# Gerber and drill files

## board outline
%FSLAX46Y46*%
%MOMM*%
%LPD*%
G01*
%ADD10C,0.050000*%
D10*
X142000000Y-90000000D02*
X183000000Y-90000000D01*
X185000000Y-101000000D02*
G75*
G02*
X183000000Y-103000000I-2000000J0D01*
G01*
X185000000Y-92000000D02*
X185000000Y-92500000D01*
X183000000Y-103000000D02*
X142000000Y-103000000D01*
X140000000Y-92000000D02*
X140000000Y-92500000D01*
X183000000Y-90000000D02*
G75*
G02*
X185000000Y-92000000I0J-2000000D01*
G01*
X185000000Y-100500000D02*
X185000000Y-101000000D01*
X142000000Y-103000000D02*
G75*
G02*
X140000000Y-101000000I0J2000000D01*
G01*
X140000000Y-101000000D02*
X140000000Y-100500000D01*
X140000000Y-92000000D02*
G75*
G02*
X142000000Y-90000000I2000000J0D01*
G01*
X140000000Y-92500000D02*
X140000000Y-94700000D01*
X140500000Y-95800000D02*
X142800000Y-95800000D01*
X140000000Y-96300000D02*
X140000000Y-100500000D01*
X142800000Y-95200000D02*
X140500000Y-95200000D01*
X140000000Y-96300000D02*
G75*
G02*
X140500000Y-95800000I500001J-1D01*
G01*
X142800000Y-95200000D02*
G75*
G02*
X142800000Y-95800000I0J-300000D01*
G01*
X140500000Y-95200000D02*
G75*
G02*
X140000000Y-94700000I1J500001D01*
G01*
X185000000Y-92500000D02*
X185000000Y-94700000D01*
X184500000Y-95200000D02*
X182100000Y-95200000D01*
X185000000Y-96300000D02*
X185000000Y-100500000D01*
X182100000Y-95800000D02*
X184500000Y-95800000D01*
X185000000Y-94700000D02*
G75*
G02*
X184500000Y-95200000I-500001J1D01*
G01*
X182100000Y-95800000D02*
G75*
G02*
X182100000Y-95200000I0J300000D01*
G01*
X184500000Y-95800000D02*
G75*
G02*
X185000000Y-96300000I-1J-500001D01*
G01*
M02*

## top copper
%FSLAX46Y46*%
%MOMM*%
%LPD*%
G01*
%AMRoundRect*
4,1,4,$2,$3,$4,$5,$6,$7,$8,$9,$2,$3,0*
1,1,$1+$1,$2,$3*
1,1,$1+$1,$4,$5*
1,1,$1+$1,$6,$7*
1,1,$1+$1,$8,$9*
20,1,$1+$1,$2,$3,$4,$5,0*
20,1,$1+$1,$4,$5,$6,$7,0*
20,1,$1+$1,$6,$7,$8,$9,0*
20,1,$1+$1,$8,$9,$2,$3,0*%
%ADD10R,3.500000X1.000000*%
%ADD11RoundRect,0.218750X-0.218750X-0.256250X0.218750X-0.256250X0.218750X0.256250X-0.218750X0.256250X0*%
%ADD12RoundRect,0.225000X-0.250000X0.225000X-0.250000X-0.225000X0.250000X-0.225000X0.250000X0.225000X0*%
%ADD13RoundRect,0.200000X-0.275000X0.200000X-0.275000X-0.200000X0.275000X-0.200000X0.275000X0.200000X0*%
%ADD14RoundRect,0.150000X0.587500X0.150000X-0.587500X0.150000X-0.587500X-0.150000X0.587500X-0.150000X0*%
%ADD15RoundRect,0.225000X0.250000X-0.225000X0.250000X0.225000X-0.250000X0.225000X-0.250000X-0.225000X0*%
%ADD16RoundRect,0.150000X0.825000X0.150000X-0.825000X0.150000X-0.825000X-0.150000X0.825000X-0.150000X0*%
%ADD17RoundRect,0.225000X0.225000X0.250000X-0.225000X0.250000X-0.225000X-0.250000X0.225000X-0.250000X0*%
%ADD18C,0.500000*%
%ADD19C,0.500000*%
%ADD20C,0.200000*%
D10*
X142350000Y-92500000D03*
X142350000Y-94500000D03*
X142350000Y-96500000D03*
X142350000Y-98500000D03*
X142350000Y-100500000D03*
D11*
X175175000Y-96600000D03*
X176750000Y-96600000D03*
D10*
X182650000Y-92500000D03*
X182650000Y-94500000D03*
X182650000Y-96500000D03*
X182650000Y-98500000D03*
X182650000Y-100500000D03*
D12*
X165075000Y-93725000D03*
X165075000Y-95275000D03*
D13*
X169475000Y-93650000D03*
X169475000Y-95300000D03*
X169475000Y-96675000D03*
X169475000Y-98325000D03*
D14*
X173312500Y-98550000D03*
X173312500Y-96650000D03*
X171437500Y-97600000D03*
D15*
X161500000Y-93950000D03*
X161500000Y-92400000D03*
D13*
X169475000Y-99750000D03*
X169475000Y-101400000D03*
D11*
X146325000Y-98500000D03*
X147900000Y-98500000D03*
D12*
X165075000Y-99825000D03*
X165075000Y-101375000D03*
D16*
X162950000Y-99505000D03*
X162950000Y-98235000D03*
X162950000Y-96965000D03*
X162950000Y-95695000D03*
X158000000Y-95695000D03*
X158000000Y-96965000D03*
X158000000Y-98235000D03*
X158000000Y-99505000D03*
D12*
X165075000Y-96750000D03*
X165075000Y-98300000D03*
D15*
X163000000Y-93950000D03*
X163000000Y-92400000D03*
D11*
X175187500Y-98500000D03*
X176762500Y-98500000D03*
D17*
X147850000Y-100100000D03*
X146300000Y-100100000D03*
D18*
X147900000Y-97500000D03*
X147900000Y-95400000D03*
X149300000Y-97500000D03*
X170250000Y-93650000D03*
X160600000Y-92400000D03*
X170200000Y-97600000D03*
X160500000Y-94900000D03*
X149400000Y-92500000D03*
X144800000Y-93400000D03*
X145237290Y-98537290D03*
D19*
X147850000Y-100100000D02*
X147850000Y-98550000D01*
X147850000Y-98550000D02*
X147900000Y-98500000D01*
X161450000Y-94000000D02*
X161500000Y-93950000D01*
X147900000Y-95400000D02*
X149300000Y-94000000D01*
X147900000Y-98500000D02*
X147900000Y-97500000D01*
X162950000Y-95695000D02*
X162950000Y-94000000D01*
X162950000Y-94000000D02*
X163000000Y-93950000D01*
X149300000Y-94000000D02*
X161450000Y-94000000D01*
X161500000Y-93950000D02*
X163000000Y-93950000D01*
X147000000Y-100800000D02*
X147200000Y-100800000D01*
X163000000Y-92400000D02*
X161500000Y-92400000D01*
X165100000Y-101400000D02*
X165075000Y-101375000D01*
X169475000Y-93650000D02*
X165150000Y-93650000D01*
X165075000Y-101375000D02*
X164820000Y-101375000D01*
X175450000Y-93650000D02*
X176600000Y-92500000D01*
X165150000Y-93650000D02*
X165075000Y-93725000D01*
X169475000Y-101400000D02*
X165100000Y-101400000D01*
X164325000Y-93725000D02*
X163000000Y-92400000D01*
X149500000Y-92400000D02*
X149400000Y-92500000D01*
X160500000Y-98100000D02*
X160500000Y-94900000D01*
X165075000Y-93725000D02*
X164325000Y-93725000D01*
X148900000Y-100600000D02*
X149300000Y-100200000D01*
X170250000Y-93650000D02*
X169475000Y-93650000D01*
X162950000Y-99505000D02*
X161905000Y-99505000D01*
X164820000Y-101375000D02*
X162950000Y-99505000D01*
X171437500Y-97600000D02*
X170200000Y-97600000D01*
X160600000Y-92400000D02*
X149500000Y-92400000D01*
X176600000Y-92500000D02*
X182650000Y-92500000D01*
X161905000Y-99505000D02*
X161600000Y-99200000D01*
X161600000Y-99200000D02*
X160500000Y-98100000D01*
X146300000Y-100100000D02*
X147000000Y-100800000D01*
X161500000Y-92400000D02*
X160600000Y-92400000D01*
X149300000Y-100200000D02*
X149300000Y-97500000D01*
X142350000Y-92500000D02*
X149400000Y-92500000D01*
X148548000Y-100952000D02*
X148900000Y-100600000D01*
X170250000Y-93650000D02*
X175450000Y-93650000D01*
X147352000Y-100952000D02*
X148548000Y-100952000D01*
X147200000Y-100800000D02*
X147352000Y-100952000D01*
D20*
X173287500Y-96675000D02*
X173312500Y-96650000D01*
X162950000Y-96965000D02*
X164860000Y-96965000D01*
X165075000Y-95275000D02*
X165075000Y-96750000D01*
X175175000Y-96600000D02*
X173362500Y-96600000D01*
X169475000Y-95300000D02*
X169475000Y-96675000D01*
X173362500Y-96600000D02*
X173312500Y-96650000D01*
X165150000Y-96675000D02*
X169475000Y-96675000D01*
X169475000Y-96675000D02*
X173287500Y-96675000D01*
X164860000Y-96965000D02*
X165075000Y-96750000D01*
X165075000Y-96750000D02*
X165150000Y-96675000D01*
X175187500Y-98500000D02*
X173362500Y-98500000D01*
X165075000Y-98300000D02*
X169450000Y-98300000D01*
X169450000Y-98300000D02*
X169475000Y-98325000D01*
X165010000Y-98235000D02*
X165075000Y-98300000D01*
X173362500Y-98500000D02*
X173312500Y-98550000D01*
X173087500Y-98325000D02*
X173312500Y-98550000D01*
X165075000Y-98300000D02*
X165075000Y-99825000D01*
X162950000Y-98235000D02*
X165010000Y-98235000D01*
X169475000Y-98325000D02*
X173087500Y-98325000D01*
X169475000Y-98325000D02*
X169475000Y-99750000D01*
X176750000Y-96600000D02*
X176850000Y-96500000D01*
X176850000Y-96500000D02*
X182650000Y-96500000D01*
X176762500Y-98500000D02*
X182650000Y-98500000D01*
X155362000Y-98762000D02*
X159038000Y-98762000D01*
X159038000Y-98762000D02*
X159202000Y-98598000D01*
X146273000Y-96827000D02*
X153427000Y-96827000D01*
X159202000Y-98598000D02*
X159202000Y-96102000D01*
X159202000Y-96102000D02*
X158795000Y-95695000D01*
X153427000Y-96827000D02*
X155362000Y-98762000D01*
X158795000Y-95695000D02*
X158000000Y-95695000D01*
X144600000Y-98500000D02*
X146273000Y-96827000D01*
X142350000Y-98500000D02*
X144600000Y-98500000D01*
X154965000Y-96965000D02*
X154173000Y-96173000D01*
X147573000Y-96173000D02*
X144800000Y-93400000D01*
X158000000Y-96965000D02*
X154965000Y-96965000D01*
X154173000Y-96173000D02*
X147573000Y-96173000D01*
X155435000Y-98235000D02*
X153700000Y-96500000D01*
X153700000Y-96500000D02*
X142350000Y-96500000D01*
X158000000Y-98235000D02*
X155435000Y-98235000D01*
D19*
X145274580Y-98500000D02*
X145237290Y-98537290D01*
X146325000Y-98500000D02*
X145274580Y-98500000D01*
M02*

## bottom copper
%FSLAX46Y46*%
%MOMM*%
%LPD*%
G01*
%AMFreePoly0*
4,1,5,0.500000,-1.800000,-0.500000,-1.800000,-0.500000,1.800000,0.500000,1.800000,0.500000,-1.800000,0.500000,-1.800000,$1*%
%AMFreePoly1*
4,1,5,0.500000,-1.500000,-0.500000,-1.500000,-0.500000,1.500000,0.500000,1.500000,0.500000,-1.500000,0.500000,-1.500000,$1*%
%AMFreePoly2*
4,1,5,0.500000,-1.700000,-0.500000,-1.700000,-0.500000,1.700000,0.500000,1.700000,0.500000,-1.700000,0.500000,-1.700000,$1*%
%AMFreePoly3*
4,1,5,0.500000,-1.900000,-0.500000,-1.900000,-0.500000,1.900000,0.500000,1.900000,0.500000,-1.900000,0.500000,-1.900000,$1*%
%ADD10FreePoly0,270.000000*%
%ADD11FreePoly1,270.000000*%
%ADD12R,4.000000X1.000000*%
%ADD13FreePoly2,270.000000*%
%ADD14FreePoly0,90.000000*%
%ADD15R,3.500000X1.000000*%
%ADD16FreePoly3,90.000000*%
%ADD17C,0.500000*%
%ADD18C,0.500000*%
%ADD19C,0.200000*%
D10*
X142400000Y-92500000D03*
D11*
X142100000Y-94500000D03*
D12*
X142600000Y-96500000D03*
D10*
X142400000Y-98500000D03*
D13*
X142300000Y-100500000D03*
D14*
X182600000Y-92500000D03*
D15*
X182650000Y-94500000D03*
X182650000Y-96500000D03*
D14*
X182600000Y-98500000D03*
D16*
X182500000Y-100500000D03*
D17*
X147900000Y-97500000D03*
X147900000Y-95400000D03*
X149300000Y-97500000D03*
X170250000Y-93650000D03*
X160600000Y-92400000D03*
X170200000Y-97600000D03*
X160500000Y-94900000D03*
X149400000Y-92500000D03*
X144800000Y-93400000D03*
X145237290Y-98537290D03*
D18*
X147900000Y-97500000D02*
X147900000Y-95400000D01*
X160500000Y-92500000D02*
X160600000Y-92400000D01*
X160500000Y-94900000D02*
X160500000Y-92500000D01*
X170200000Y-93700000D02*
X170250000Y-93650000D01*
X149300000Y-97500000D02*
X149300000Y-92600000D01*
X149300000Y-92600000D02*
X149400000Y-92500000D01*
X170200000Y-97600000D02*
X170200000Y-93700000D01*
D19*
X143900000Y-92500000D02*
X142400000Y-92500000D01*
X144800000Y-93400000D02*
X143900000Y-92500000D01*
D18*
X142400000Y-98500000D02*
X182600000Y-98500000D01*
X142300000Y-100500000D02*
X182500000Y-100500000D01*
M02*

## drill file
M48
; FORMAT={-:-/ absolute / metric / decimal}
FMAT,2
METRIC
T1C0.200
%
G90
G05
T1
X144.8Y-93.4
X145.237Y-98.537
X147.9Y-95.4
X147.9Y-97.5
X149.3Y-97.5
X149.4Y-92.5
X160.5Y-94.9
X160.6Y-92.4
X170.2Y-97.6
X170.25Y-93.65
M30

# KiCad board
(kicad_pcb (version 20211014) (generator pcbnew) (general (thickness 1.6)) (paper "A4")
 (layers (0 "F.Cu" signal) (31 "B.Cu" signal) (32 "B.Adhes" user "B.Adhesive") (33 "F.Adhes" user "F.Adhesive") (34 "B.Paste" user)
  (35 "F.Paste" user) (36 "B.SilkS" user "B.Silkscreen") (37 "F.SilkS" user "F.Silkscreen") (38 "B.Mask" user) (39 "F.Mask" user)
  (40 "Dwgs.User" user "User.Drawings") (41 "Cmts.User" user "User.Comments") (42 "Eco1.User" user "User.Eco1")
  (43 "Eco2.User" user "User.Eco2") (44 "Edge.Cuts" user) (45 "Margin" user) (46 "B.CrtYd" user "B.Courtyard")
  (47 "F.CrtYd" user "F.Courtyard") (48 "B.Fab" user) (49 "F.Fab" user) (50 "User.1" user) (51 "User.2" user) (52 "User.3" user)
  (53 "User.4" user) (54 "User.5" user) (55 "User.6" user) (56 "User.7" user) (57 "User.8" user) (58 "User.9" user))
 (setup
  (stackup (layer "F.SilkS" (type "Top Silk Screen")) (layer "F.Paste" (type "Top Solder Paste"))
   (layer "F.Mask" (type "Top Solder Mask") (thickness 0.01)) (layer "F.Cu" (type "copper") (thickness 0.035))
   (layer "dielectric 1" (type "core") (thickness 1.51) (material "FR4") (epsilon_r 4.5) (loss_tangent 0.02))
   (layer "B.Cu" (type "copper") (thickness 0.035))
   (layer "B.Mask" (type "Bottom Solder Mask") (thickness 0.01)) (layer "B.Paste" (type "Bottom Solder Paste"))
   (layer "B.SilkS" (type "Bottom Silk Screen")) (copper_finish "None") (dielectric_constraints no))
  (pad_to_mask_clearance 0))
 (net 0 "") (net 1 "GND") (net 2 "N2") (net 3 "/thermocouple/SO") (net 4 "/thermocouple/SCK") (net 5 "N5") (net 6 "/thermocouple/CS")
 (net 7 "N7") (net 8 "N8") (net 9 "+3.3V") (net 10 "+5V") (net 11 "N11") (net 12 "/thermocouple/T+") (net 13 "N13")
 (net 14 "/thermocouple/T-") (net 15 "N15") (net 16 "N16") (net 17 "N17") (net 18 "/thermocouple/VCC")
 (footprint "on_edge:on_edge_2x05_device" (layer "F.Cu") (at 140 96.5 -90)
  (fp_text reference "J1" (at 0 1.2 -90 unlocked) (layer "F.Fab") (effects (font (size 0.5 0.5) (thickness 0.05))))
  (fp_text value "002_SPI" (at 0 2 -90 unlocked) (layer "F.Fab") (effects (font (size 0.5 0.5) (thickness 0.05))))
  (fp_line (start -4 0) (end -1.8 0) (layer "Edge.Cuts") (width 0.05))
  (fp_line (start -0.7 -0.5) (end -0.7 -2.8) (layer "Edge.Cuts") (width 0.05))
  (fp_line (start -0.2 0) (end 4 0) (layer "Edge.Cuts") (width 0.05))
  (fp_line (start -1.3 -2.8) (end -1.3 -0.5) (layer "Edge.Cuts") (width 0.05))
  (fp_arc (start -0.2 0) (mid -0.553553 -0.146447) (end -0.7 -0.5) (layer "Edge.Cuts") (width 0.05))
  (fp_arc (start -1.3 -2.8) (mid -1 -3.1) (end -0.7 -2.8) (layer "Edge.Cuts") (width 0.05))
  (fp_arc (start -1.3 -0.5) (mid -1.446447 -0.146447) (end -1.8 0) (layer "Edge.Cuts") (width 0.05))
  (pad "1" smd rect (at -4 -2.35 90) (size 1 3.5) (layers "F.Cu" "F.Mask") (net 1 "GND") (zone_connect 0))
  (pad "2" smd rect (at -2 -2.35 270) (size 1 3.5) (layers "F.Cu" "F.Mask") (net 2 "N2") (zone_connect 0))
  (pad "3" smd rect (at 0 -2.35 270) (size 1 3.5) (layers "F.Cu" "F.Mask") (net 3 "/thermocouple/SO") (zone_connect 0))
  (pad "4" smd rect (at 2 -2.35 90) (size 1 3.5) (layers "F.Cu" "F.Mask") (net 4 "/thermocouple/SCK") (zone_connect 0))
  (pad "5" smd rect (at 4 -2.35 90) (size 1 3.5) (layers "F.Cu" "F.Mask") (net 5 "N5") (zone_connect 0))
  (pad "6" smd custom (at -4 -2.4 270) (size 1 3.6) (layers "B.Cu" "B.Mask") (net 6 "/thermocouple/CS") (zone_connect 0)
   (options (clearance outline) (anchor rect)) (primitives))
  (pad "7" smd custom (at -2 -2.1 270) (size 1 3) (layers "B.Cu" "B.Mask") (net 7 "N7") (zone_connect 0)
   (options (clearance outline) (anchor rect)) (primitives))
  (pad "8" smd rect (at 0 -2.6 270) (size 1 4) (layers "B.Cu" "B.Mask") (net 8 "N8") (zone_connect 0))
  (pad "9" smd custom (at 2 -2.4 270) (size 1 3.6) (layers "B.Cu" "B.Mask") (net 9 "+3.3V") (zone_connect 0)
   (options (clearance outline) (anchor rect)) (primitives))
  (pad "10" smd custom (at 4 -2.3 270) (size 1 3.4) (layers "B.Cu" "B.Mask") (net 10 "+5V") (zone_connect 0)
   (options (clearance outline) (anchor rect)) (primitives))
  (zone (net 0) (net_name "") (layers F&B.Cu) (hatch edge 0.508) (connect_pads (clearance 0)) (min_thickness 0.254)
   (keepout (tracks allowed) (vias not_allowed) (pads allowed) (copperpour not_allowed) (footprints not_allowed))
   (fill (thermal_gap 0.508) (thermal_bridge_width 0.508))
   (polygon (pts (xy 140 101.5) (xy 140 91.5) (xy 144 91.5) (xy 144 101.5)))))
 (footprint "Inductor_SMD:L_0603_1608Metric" (layer "F.Cu") (at 175.9625 96.6)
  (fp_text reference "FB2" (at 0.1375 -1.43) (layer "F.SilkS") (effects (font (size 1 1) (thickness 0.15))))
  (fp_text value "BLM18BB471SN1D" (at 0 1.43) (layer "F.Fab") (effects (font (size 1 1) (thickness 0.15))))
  (pad "1" smd roundrect (at -0.7875 0) (size 0.875 0.95) (layers "F.Cu" "F.Paste" "F.Mask") (roundrect_rratio 0.25) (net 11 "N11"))
  (pad "2" smd roundrect (at 0.7875 0) (size 0.875 0.95) (layers "F.Cu" "F.Paste" "F.Mask") (roundrect_rratio 0.25)
   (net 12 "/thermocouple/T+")))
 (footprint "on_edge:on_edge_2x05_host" (layer "F.Cu") (at 185 96.5 -90)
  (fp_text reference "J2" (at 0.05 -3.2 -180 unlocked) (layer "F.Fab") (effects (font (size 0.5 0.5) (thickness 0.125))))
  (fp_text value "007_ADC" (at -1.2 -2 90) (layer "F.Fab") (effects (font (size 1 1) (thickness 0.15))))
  (fp_line (start -4 0) (end -1.8 0) (layer "Edge.Cuts") (width 0.05))
  (fp_line (start -1.3 0.5) (end -1.3 2.9) (layer "Edge.Cuts") (width 0.05))
  (fp_line (start -0.2 0) (end 4 0) (layer "Edge.Cuts") (width 0.05))
  (fp_line (start -0.7 2.9) (end -0.7 0.5) (layer "Edge.Cuts") (width 0.05))
  (fp_arc (start -1.8 0) (mid -1.446447 0.146447) (end -1.3 0.5) (layer "Edge.Cuts") (width 0.05))
  (fp_arc (start -0.7 2.9) (mid -1 3.2) (end -1.3 2.9) (layer "Edge.Cuts") (width 0.05))
  (fp_arc (start -0.7 0.5) (mid -0.553553 0.146447) (end -0.2 0) (layer "Edge.Cuts") (width 0.05))
  (pad "1" smd rect (at -4 2.35 270) (size 1 3.5) (layers "F.Cu" "F.Mask") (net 1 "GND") (zone_connect 0))
  (pad "2" smd rect (at -2 2.35 270) (size 1 3.5) (layers "F.Cu" "F.Mask") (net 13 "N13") (zone_connect 0))
  (pad "3" smd rect (at 0 2.35 270) (size 1 3.5) (layers "F.Cu" "F.Mask") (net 12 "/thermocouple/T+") (zone_connect 0))
  (pad "4" smd rect (at 2 2.35 270) (size 1 3.5) (layers "F.Cu" "F.Mask") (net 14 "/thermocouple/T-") (zone_connect 0))
  (pad "5" smd rect (at 4 2.35 270) (size 1 3.5) (layers "F.Cu" "F.Mask") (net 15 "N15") (zone_connect 0))
  (pad "6" smd custom (at -4 2.4 90) (size 1 3.6) (layers "B.Cu" "B.Mask") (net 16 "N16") (zone_connect 0)
   (options (clearance outline) (anchor rect)) (primitives))
  (pad "7" smd rect (at -2 2.35 90) (size 1 3.5) (layers "B.Cu" "B.Mask") (zone_connect 0))
  (pad "8" smd rect (at 0 2.35 90) (size 1 3.5) (layers "B.Cu" "B.Mask") (zone_connect 0))
  (pad "9" smd custom (at 2 2.4 90) (size 1 3.6) (layers "B.Cu" "B.Mask") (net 9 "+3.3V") (zone_connect 0)
   (options (clearance outline) (anchor rect)) (primitives))
  (pad "10" smd custom (at 4 2.5 90) (size 1 3.8) (layers "B.Cu" "B.Mask") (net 10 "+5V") (zone_connect 0)
   (options (clearance outline) (anchor rect)) (primitives))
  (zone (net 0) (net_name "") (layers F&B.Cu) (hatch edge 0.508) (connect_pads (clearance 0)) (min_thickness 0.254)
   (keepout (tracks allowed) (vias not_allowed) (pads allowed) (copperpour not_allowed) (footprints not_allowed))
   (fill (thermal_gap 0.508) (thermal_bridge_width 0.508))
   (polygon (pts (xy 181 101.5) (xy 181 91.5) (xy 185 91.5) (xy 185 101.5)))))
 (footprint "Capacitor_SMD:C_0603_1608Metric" (layer "F.Cu") (at 165.075 94.5 -90)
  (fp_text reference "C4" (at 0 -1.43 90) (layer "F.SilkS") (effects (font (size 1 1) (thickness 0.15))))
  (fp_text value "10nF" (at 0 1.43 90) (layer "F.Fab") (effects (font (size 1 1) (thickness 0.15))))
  (pad "1" smd roundrect (at -0.775 0 270) (size 0.9 0.95) (layers "F.Cu" "F.Paste" "F.Mask") (roundrect_rratio 0.25) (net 1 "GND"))
  (pad "2" smd roundrect (at 0.775 0 270) (size 0.9 0.95) (layers "F.Cu" "F.Paste" "F.Mask") (roundrect_rratio 0.25) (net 11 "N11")))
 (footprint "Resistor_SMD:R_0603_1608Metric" (layer "F.Cu") (at 169.475 94.475 -90)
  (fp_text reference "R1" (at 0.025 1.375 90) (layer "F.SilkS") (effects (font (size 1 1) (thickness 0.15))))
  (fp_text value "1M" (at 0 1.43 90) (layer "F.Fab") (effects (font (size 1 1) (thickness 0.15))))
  (pad "1" smd roundrect (at -0.825 0 270) (size 0.8 0.95) (layers "F.Cu" "F.Paste" "F.Mask") (roundrect_rratio 0.25) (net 1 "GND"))
  (pad "2" smd roundrect (at 0.825 0 270) (size 0.8 0.95) (layers "F.Cu" "F.Paste" "F.Mask") (roundrect_rratio 0.25) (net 11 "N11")))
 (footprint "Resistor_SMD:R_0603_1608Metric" (layer "F.Cu") (at 169.475 97.5 -90)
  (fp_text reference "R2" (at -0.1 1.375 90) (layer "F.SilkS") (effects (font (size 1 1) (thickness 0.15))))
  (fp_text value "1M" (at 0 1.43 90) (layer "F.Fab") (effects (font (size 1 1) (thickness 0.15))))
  (pad "1" smd roundrect (at -0.825 0 270) (size 0.8 0.95) (layers "F.Cu" "F.Paste" "F.Mask") (roundrect_rratio 0.25) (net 11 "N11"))
  (pad "2" smd roundrect (at 0.825 0 270) (size 0.8 0.95) (layers "F.Cu" "F.Paste" "F.Mask") (roundrect_rratio 0.25) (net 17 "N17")))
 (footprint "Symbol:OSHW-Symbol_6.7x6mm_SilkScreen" (layer "F.Cu") (at 152.8 99.2)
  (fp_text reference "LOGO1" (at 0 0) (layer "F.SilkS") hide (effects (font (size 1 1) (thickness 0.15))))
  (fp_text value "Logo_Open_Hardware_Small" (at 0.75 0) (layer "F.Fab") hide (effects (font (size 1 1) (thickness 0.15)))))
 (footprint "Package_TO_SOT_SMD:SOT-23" (layer "F.Cu") (at 172.375 97.6 180)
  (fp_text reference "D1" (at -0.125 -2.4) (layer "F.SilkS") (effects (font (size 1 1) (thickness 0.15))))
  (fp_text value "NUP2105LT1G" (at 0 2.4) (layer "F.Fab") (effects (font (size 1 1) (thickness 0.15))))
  (pad "1" smd roundrect (at -0.9375 -0.95 180) (size 1.475 0.6) (layers "F.Cu" "F.Paste" "F.Mask") (roundrect_rratio 0.25) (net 17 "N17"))
  (pad "2" smd roundrect (at -0.9375 0.95 180) (size 1.475 0.6) (layers "F.Cu" "F.Paste" "F.Mask") (roundrect_rratio 0.25) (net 11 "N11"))
  (pad "3" smd roundrect (at 0.9375 0 180) (size 1.475 0.6) (layers "F.Cu" "F.Paste" "F.Mask") (roundrect_rratio 0.25) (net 1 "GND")))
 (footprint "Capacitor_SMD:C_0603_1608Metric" (layer "F.Cu") (at 161.5 93.175 90)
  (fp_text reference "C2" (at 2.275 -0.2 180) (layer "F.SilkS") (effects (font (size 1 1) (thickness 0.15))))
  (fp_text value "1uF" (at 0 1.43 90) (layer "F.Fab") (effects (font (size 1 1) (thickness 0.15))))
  (pad "1" smd roundrect (at -0.775 0 90) (size 0.9 0.95) (layers "F.Cu" "F.Paste" "F.Mask") (roundrect_rratio 0.25)
   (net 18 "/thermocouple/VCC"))
  (pad "2" smd roundrect (at 0.775 0 90) (size 0.9 0.95) (layers "F.Cu" "F.Paste" "F.Mask") (roundrect_rratio 0.25) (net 1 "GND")))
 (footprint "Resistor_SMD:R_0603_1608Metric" (layer "F.Cu") (at 169.475 100.575 -90)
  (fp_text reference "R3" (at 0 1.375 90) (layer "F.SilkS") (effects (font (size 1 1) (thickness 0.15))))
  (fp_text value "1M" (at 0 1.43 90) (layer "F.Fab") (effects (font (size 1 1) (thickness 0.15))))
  (pad "1" smd roundrect (at -0.825 0 270) (size 0.8 0.95) (layers "F.Cu" "F.Paste" "F.Mask") (roundrect_rratio 0.25) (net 17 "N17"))
  (pad "2" smd roundrect (at 0.825 0 270) (size 0.8 0.95) (layers "F.Cu" "F.Paste" "F.Mask") (roundrect_rratio 0.25) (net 1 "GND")))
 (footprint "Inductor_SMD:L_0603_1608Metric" (layer "F.Cu") (at 147.1125 98.5)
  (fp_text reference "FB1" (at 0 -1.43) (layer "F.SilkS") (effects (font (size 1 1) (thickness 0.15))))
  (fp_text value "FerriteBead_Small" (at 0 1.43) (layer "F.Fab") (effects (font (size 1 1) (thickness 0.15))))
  (pad "1" smd roundrect (at -0.7875 0) (size 0.875 0.95) (layers "F.Cu" "F.Paste" "F.Mask") (roundrect_rratio 0.25) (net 9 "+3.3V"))
  (pad "2" smd roundrect (at 0.7875 0) (size 0.875 0.95) (layers "F.Cu" "F.Paste" "F.Mask") (roundrect_rratio 0.25)
   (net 18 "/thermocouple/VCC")))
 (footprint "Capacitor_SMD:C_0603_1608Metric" (layer "F.Cu") (at 165.075 100.6 -90)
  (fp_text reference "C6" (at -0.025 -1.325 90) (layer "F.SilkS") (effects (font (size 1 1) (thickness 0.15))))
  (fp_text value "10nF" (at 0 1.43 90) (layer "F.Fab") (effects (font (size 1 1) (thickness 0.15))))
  (pad "1" smd roundrect (at -0.775 0 270) (size 0.9 0.95) (layers "F.Cu" "F.Paste" "F.Mask") (roundrect_rratio 0.25) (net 17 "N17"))
  (pad "2" smd roundrect (at 0.775 0 270) (size 0.9 0.95) (layers "F.Cu" "F.Paste" "F.Mask") (roundrect_rratio 0.25) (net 1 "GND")))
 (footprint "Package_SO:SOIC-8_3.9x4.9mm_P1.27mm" (layer "F.Cu") (at 160.475 97.6 180)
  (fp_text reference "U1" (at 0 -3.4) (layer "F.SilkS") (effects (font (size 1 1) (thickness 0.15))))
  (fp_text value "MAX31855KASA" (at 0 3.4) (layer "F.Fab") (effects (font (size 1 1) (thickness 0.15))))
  (pad "1" smd roundrect (at -2.475 -1.905 180) (size 1.95 0.6) (layers "F.Cu" "F.Paste" "F.Mask") (roundrect_rratio 0.25) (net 1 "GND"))
  (pad "2" smd roundrect (at -2.475 -0.635 180) (size 1.95 0.6) (layers "F.Cu" "F.Paste" "F.Mask") (roundrect_rratio 0.25) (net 17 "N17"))
  (pad "3" smd roundrect (at -2.475 0.635 180) (size 1.95 0.6) (layers "F.Cu" "F.Paste" "F.Mask") (roundrect_rratio 0.25) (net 11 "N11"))
  (pad "4" smd roundrect (at -2.475 1.905 180) (size 1.95 0.6) (layers "F.Cu" "F.Paste" "F.Mask") (roundrect_rratio 0.25)
   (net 18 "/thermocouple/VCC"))
  (pad "5" smd roundrect (at 2.475 1.905 180) (size 1.95 0.6) (layers "F.Cu" "F.Paste" "F.Mask") (roundrect_rratio 0.25)
   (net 4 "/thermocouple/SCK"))
  (pad "6" smd roundrect (at 2.475 0.635 180) (size 1.95 0.6) (layers "F.Cu" "F.Paste" "F.Mask") (roundrect_rratio 0.25)
   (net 6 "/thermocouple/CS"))
  (pad "7" smd roundrect (at 2.475 -0.635 180) (size 1.95 0.6) (layers "F.Cu" "F.Paste" "F.Mask") (roundrect_rratio 0.25)
   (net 3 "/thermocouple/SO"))
  (pad "8" smd roundrect (at 2.475 -1.905 180) (size 1.95 0.6) (layers "F.Cu" "F.Paste" "F.Mask") (roundrect_rratio 0.25)))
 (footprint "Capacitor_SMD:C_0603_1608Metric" (layer "F.Cu") (at 165.075 97.525 -90)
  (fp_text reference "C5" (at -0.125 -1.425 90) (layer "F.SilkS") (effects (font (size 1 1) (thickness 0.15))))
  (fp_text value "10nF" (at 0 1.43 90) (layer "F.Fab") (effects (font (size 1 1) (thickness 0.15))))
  (pad "1" smd roundrect (at -0.775 0 270) (size 0.9 0.95) (layers "F.Cu" "F.Paste" "F.Mask") (roundrect_rratio 0.25) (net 11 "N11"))
  (pad "2" smd roundrect (at 0.775 0 270) (size 0.9 0.95) (layers "F.Cu" "F.Paste" "F.Mask") (roundrect_rratio 0.25) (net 17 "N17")))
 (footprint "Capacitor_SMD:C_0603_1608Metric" (layer "F.Cu") (at 163 93.175 90)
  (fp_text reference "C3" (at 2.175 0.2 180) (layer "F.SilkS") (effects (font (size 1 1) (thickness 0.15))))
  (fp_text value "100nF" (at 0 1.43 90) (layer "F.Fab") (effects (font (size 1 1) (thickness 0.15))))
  (pad "1" smd roundrect (at -0.775 0 90) (size 0.9 0.95) (layers "F.Cu" "F.Paste" "F.Mask") (roundrect_rratio 0.25)
   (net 18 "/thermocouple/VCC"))
  (pad "2" smd roundrect (at 0.775 0 90) (size 0.9 0.95) (layers "F.Cu" "F.Paste" "F.Mask") (roundrect_rratio 0.25) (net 1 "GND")))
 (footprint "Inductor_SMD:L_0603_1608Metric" (layer "F.Cu") (at 175.975 98.5)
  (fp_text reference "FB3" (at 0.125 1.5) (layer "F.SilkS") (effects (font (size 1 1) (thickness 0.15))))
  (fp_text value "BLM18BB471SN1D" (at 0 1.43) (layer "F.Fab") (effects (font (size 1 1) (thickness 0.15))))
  (pad "1" smd roundrect (at -0.7875 0) (size 0.875 0.95) (layers "F.Cu" "F.Paste" "F.Mask") (roundrect_rratio 0.25) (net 17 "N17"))
  (pad "2" smd roundrect (at 0.7875 0) (size 0.875 0.95) (layers "F.Cu" "F.Paste" "F.Mask") (roundrect_rratio 0.25)
   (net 14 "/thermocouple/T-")))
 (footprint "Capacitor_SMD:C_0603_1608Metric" (layer "F.Cu") (at 147.075 100.1 180)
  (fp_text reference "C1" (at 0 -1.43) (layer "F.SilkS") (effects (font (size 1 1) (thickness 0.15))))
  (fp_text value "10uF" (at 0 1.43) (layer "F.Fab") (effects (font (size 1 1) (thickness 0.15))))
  (pad "1" smd roundrect (at -0.775 0 180) (size 0.9 0.95) (layers "F.Cu" "F.Paste" "F.Mask") (roundrect_rratio 0.25)
   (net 18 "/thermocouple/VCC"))
  (pad "2" smd roundrect (at 0.775 0 180) (size 0.9 0.95) (layers "F.Cu" "F.Paste" "F.Mask") (roundrect_rratio 0.25) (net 1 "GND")))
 (gr_line (start 142 90) (end 183 90) (layer "Edge.Cuts") (width 0.05))
 (gr_arc (start 185 101) (mid 184.414214 102.414214) (end 183 103) (layer "Edge.Cuts") (width 0.05))
 (gr_line (start 185 92) (end 185 92.5) (layer "Edge.Cuts") (width 0.05))
 (gr_line (start 183 103) (end 142 103) (layer "Edge.Cuts") (width 0.05))
 (gr_line (start 140 92) (end 140 92.5) (layer "Edge.Cuts") (width 0.05))
 (gr_arc (start 183 90) (mid 184.414214 90.585786) (end 185 92) (layer "Edge.Cuts") (width 0.05))
 (gr_line (start 185 100.5) (end 185 101) (layer "Edge.Cuts") (width 0.05))
 (gr_arc (start 142 103) (mid 140.585786 102.414214) (end 140 101) (layer "Edge.Cuts") (width 0.05))
 (gr_line (start 140 101) (end 140 100.5) (layer "Edge.Cuts") (width 0.05))
 (gr_arc (start 140 92) (mid 140.585786 90.585786) (end 142 90) (layer "Edge.Cuts") (width 0.05))
 (segment (start 147.85 100.1) (end 147.85 98.55) (width 0.5) (layer "F.Cu") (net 18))
 (segment (start 147.85 98.55) (end 147.9 98.5) (width 0.5) (layer "F.Cu") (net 18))
 (segment (start 161.45 94) (end 161.5 93.95) (width 0.5) (layer "F.Cu") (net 18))
 (segment (start 147.9 95.4) (end 149.3 94) (width 0.5) (layer "F.Cu") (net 18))
 (segment (start 147.9 98.5) (end 147.9 97.5) (width 0.5) (layer "F.Cu") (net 18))
 (segment (start 162.95 95.695) (end 162.95 94) (width 0.5) (layer "F.Cu") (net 18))
 (segment (start 162.95 94) (end 163 93.95) (width 0.5) (layer "F.Cu") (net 18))
 (segment (start 149.3 94) (end 161.45 94) (width 0.5) (layer "F.Cu") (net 18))
 (segment (start 161.5 93.95) (end 163 93.95) (width 0.5) (layer "F.Cu") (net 18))
 (via (at 147.9 97.5) (size 0.5) (drill 0.2) (layers "F.Cu" "B.Cu") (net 18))
 (via (at 147.9 95.4) (size 0.5) (drill 0.2) (layers "F.Cu" "B.Cu") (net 18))
 (segment (start 147.9 97.5) (end 147.9 95.4) (width 0.5) (layer "B.Cu") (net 18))
 (segment (start 147 100.8) (end 147.2 100.8) (width 0.5) (layer "F.Cu") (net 1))
 (segment (start 163 92.4) (end 161.5 92.4) (width 0.5) (layer "F.Cu") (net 1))
 (segment (start 165.1 101.4) (end 165.075 101.375) (width 0.5) (layer "F.Cu") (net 1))
 (segment (start 169.475 93.65) (end 165.15 93.65) (width 0.5) (layer "F.Cu") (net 1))
 (segment (start 165.075 101.375) (end 164.82 101.375) (width 0.5) (layer "F.Cu") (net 1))
 (segment (start 175.45 93.65) (end 176.6 92.5) (width 0.5) (layer "F.Cu") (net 1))
 (segment (start 165.15 93.65) (end 165.075 93.725) (width 0.5) (layer "F.Cu") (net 1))
 (segment (start 169.475 101.4) (end 165.1 101.4) (width 0.5) (layer "F.Cu") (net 1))
 (segment (start 164.325 93.725) (end 163 92.4) (width 0.5) (layer "F.Cu") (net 1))
 (segment (start 149.5 92.4) (end 149.4 92.5) (width 0.5) (layer "F.Cu") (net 1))
 (segment (start 160.5 98.1) (end 160.5 94.9) (width 0.5) (layer "F.Cu") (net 1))
 (segment (start 165.075 93.725) (end 164.325 93.725) (width 0.5) (layer "F.Cu") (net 1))
 (segment (start 148.9 100.6) (end 149.3 100.2) (width 0.5) (layer "F.Cu") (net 1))
 (segment (start 170.25 93.65) (end 169.475 93.65) (width 0.5) (layer "F.Cu") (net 1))
 (segment (start 162.95 99.505) (end 161.905 99.505) (width 0.5) (layer "F.Cu") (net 1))
 (segment (start 164.82 101.375) (end 162.95 99.505) (width 0.5) (layer "F.Cu") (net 1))
 (segment (start 171.4375 97.6) (end 170.2 97.6) (width 0.5) (layer "F.Cu") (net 1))
 (segment (start 160.6 92.4) (end 149.5 92.4) (width 0.5) (layer "F.Cu") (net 1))
 (segment (start 176.6 92.5) (end 182.65 92.5) (width 0.5) (layer "F.Cu") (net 1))
 (segment (start 161.905 99.505) (end 161.6 99.2) (width 0.5) (layer "F.Cu") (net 1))
 (segment (start 161.6 99.2) (end 160.5 98.1) (width 0.5) (layer "F.Cu") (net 1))
 (segment (start 146.3 100.1) (end 147 100.8) (width 0.5) (layer "F.Cu") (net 1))
 (segment (start 161.5 92.4) (end 160.6 92.4) (width 0.5) (layer "F.Cu") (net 1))
 (segment (start 149.3 100.2) (end 149.3 97.5) (width 0.5) (layer "F.Cu") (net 1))
 (segment (start 142.35 92.5) (end 149.4 92.5) (width 0.5) (layer "F.Cu") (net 1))
 (segment (start 148.548 100.952) (end 148.9 100.6) (width 0.5) (layer "F.Cu") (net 1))
 (segment (start 170.25 93.65) (end 175.45 93.65) (width 0.5) (layer "F.Cu") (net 1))
 (segment (start 147.352 100.952) (end 148.548 100.952) (width 0.5) (layer "F.Cu") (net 1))
 (segment (start 147.2 100.8) (end 147.352 100.952) (width 0.5) (layer "F.Cu") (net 1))
 (via (at 149.3 97.5) (size 0.5) (drill 0.2) (layers "F.Cu" "B.Cu") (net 1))
 (via (at 170.25 93.65) (size 0.5) (drill 0.2) (layers "F.Cu" "B.Cu") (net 1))
 (via (at 160.6 92.4) (size 0.5) (drill 0.2) (layers "F.Cu" "B.Cu") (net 1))
 (via (at 170.2 97.6) (size 0.5) (drill 0.2) (layers "F.Cu" "B.Cu") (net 1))
 (via (at 160.5 94.9) (size 0.5) (drill 0.2) (layers "F.Cu" "B.Cu") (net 1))
 (via (at 149.4 92.5) (size 0.5) (drill 0.2) (layers "F.Cu" "B.Cu") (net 1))
 (segment (start 160.5 92.5) (end 160.6 92.4) (width 0.5) (layer "B.Cu") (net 1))
 (segment (start 160.5 94.9) (end 160.5 92.5) (width 0.5) (layer "B.Cu") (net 1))
 (segment (start 170.2 93.7) (end 170.25 93.65) (width 0.5) (layer "B.Cu") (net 1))
 (segment (start 149.3 97.5) (end 149.3 92.6) (width 0.5) (layer "B.Cu") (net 1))
 (segment (start 149.3 92.6) (end 149.4 92.5) (width 0.5) (layer "B.Cu") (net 1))
 (segment (start 170.2 97.6) (end 170.2 93.7) (width 0.5) (layer "B.Cu") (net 1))
 (segment (start 173.2875 96.675) (end 173.3125 96.65) (width 0.2) (layer "F.Cu") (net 11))
 (segment (start 162.95 96.965) (end 164.86 96.965) (width 0.2) (layer "F.Cu") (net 11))
 (segment (start 165.075 95.275) (end 165.075 96.75) (width 0.2) (layer "F.Cu") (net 11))
 (segment (start 175.175 96.6) (end 173.3625 96.6) (width 0.2) (layer "F.Cu") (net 11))
 (segment (start 169.475 95.3) (end 169.475 96.675) (width 0.2) (layer "F.Cu") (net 11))
 (segment (start 173.3625 96.6) (end 173.3125 96.65) (width 0.2) (layer "F.Cu") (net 11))
 (segment (start 165.15 96.675) (end 169.475 96.675) (width 0.2) (layer "F.Cu") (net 11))
 (segment (start 169.475 96.675) (end 173.2875 96.675) (width 0.2) (layer "F.Cu") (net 11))
 (segment (start 164.86 96.965) (end 165.075 96.75) (width 0.2) (layer "F.Cu") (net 11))
 (segment (start 165.075 96.75) (end 165.15 96.675) (width 0.2) (layer "F.Cu") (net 11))
 (segment (start 175.1875 98.5) (end 173.3625 98.5) (width 0.2) (layer "F.Cu") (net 17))
 (segment (start 165.075 98.3) (end 169.45 98.3) (width 0.2) (layer "F.Cu") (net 17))
 (segment (start 169.45 98.3) (end 169.475 98.325) (width 0.2) (layer "F.Cu") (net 17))
 (segment (start 165.01 98.235) (end 165.075 98.3) (width 0.2) (layer "F.Cu") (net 17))
 (segment (start 173.3625 98.5) (end 173.3125 98.55) (width 0.2) (layer "F.Cu") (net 17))
 (segment (start 173.0875 98.325) (end 173.3125 98.55) (width 0.2) (layer "F.Cu") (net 17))
 (segment (start 165.075 98.3) (end 165.075 99.825) (width 0.2) (layer "F.Cu") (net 17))
 (segment (start 162.95 98.235) (end 165.01 98.235) (width 0.2) (layer "F.Cu") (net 17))
 (segment (start 169.475 98.325) (end 173.0875 98.325) (width 0.2) (layer "F.Cu") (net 17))
 (segment (start 169.475 98.325) (end 169.475 99.75) (width 0.2) (layer "F.Cu") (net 17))
 (segment (start 176.75 96.6) (end 176.85 96.5) (width 0.2) (layer "F.Cu") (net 12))
 (segment (start 176.85 96.5) (end 182.65 96.5) (width 0.2) (layer "F.Cu") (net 12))
 (segment (start 176.7625 98.5) (end 182.65 98.5) (width 0.2) (layer "F.Cu") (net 14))
 (segment (start 155.362 98.762) (end 159.038 98.762) (width 0.2) (layer "F.Cu") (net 4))
 (segment (start 159.038 98.762) (end 159.202 98.598) (width 0.2) (layer "F.Cu") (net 4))
 (segment (start 146.273 96.827) (end 153.427 96.827) (width 0.2) (layer "F.Cu") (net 4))
 (segment (start 159.202 98.598) (end 159.202 96.102) (width 0.2) (layer "F.Cu") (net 4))
 (segment (start 159.202 96.102) (end 158.795 95.695) (width 0.2) (layer "F.Cu") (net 4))
 (segment (start 153.427 96.827) (end 155.362 98.762) (width 0.2) (layer "F.Cu") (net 4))
 (segment (start 158.795 95.695) (end 158 95.695) (width 0.2) (layer "F.Cu") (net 4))
 (segment (start 144.6 98.5) (end 146.273 96.827) (width 0.2) (layer "F.Cu") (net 4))
 (segment (start 142.35 98.5) (end 144.6 98.5) (width 0.2) (layer "F.Cu") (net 4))
 (segment (start 154.965 96.965) (end 154.173 96.173) (width 0.2) (layer "F.Cu") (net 6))
 (segment (start 147.573 96.173) (end 144.8 93.4) (width 0.2) (layer "F.Cu") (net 6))
 (segment (start 158 96.965) (end 154.965 96.965) (width 0.2) (layer "F.Cu") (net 6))
 (segment (start 154.173 96.173) (end 147.573 96.173) (width 0.2) (layer "F.Cu") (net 6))
 (via (at 144.8 93.4) (size 0.5) (drill 0.2) (layers "F.Cu" "B.Cu") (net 6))
 (segment (start 143.9 92.5) (end 142.4 92.5) (width 0.2) (layer "B.Cu") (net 6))
 (segment (start 144.8 93.4) (end 143.9 92.5) (width 0.2) (layer "B.Cu") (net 6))
 (segment (start 155.435 98.235) (end 153.7 96.5) (width 0.2) (layer "F.Cu") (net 3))
 (segment (start 153.7 96.5) (end 142.35 96.5) (width 0.2) (layer "F.Cu") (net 3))
 (segment (start 158 98.235) (end 155.435 98.235) (width 0.2) (layer "F.Cu") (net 3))
 (segment (start 145.27458 98.5) (end 145.23729 98.53729) (width 0.5) (layer "F.Cu") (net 9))
 (segment (start 146.325 98.5) (end 145.27458 98.5) (width 0.5) (layer "F.Cu") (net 9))
 (via (at 145.23729 98.53729) (size 0.5) (drill 0.2) (layers "F.Cu" "B.Cu") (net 9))
 (segment (start 142.4 98.5) (end 182.6 98.5) (width 0.5) (layer "B.Cu") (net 9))
 (segment (start 142.3 100.5) (end 182.5 100.5) (width 0.5) (layer "B.Cu") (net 10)))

